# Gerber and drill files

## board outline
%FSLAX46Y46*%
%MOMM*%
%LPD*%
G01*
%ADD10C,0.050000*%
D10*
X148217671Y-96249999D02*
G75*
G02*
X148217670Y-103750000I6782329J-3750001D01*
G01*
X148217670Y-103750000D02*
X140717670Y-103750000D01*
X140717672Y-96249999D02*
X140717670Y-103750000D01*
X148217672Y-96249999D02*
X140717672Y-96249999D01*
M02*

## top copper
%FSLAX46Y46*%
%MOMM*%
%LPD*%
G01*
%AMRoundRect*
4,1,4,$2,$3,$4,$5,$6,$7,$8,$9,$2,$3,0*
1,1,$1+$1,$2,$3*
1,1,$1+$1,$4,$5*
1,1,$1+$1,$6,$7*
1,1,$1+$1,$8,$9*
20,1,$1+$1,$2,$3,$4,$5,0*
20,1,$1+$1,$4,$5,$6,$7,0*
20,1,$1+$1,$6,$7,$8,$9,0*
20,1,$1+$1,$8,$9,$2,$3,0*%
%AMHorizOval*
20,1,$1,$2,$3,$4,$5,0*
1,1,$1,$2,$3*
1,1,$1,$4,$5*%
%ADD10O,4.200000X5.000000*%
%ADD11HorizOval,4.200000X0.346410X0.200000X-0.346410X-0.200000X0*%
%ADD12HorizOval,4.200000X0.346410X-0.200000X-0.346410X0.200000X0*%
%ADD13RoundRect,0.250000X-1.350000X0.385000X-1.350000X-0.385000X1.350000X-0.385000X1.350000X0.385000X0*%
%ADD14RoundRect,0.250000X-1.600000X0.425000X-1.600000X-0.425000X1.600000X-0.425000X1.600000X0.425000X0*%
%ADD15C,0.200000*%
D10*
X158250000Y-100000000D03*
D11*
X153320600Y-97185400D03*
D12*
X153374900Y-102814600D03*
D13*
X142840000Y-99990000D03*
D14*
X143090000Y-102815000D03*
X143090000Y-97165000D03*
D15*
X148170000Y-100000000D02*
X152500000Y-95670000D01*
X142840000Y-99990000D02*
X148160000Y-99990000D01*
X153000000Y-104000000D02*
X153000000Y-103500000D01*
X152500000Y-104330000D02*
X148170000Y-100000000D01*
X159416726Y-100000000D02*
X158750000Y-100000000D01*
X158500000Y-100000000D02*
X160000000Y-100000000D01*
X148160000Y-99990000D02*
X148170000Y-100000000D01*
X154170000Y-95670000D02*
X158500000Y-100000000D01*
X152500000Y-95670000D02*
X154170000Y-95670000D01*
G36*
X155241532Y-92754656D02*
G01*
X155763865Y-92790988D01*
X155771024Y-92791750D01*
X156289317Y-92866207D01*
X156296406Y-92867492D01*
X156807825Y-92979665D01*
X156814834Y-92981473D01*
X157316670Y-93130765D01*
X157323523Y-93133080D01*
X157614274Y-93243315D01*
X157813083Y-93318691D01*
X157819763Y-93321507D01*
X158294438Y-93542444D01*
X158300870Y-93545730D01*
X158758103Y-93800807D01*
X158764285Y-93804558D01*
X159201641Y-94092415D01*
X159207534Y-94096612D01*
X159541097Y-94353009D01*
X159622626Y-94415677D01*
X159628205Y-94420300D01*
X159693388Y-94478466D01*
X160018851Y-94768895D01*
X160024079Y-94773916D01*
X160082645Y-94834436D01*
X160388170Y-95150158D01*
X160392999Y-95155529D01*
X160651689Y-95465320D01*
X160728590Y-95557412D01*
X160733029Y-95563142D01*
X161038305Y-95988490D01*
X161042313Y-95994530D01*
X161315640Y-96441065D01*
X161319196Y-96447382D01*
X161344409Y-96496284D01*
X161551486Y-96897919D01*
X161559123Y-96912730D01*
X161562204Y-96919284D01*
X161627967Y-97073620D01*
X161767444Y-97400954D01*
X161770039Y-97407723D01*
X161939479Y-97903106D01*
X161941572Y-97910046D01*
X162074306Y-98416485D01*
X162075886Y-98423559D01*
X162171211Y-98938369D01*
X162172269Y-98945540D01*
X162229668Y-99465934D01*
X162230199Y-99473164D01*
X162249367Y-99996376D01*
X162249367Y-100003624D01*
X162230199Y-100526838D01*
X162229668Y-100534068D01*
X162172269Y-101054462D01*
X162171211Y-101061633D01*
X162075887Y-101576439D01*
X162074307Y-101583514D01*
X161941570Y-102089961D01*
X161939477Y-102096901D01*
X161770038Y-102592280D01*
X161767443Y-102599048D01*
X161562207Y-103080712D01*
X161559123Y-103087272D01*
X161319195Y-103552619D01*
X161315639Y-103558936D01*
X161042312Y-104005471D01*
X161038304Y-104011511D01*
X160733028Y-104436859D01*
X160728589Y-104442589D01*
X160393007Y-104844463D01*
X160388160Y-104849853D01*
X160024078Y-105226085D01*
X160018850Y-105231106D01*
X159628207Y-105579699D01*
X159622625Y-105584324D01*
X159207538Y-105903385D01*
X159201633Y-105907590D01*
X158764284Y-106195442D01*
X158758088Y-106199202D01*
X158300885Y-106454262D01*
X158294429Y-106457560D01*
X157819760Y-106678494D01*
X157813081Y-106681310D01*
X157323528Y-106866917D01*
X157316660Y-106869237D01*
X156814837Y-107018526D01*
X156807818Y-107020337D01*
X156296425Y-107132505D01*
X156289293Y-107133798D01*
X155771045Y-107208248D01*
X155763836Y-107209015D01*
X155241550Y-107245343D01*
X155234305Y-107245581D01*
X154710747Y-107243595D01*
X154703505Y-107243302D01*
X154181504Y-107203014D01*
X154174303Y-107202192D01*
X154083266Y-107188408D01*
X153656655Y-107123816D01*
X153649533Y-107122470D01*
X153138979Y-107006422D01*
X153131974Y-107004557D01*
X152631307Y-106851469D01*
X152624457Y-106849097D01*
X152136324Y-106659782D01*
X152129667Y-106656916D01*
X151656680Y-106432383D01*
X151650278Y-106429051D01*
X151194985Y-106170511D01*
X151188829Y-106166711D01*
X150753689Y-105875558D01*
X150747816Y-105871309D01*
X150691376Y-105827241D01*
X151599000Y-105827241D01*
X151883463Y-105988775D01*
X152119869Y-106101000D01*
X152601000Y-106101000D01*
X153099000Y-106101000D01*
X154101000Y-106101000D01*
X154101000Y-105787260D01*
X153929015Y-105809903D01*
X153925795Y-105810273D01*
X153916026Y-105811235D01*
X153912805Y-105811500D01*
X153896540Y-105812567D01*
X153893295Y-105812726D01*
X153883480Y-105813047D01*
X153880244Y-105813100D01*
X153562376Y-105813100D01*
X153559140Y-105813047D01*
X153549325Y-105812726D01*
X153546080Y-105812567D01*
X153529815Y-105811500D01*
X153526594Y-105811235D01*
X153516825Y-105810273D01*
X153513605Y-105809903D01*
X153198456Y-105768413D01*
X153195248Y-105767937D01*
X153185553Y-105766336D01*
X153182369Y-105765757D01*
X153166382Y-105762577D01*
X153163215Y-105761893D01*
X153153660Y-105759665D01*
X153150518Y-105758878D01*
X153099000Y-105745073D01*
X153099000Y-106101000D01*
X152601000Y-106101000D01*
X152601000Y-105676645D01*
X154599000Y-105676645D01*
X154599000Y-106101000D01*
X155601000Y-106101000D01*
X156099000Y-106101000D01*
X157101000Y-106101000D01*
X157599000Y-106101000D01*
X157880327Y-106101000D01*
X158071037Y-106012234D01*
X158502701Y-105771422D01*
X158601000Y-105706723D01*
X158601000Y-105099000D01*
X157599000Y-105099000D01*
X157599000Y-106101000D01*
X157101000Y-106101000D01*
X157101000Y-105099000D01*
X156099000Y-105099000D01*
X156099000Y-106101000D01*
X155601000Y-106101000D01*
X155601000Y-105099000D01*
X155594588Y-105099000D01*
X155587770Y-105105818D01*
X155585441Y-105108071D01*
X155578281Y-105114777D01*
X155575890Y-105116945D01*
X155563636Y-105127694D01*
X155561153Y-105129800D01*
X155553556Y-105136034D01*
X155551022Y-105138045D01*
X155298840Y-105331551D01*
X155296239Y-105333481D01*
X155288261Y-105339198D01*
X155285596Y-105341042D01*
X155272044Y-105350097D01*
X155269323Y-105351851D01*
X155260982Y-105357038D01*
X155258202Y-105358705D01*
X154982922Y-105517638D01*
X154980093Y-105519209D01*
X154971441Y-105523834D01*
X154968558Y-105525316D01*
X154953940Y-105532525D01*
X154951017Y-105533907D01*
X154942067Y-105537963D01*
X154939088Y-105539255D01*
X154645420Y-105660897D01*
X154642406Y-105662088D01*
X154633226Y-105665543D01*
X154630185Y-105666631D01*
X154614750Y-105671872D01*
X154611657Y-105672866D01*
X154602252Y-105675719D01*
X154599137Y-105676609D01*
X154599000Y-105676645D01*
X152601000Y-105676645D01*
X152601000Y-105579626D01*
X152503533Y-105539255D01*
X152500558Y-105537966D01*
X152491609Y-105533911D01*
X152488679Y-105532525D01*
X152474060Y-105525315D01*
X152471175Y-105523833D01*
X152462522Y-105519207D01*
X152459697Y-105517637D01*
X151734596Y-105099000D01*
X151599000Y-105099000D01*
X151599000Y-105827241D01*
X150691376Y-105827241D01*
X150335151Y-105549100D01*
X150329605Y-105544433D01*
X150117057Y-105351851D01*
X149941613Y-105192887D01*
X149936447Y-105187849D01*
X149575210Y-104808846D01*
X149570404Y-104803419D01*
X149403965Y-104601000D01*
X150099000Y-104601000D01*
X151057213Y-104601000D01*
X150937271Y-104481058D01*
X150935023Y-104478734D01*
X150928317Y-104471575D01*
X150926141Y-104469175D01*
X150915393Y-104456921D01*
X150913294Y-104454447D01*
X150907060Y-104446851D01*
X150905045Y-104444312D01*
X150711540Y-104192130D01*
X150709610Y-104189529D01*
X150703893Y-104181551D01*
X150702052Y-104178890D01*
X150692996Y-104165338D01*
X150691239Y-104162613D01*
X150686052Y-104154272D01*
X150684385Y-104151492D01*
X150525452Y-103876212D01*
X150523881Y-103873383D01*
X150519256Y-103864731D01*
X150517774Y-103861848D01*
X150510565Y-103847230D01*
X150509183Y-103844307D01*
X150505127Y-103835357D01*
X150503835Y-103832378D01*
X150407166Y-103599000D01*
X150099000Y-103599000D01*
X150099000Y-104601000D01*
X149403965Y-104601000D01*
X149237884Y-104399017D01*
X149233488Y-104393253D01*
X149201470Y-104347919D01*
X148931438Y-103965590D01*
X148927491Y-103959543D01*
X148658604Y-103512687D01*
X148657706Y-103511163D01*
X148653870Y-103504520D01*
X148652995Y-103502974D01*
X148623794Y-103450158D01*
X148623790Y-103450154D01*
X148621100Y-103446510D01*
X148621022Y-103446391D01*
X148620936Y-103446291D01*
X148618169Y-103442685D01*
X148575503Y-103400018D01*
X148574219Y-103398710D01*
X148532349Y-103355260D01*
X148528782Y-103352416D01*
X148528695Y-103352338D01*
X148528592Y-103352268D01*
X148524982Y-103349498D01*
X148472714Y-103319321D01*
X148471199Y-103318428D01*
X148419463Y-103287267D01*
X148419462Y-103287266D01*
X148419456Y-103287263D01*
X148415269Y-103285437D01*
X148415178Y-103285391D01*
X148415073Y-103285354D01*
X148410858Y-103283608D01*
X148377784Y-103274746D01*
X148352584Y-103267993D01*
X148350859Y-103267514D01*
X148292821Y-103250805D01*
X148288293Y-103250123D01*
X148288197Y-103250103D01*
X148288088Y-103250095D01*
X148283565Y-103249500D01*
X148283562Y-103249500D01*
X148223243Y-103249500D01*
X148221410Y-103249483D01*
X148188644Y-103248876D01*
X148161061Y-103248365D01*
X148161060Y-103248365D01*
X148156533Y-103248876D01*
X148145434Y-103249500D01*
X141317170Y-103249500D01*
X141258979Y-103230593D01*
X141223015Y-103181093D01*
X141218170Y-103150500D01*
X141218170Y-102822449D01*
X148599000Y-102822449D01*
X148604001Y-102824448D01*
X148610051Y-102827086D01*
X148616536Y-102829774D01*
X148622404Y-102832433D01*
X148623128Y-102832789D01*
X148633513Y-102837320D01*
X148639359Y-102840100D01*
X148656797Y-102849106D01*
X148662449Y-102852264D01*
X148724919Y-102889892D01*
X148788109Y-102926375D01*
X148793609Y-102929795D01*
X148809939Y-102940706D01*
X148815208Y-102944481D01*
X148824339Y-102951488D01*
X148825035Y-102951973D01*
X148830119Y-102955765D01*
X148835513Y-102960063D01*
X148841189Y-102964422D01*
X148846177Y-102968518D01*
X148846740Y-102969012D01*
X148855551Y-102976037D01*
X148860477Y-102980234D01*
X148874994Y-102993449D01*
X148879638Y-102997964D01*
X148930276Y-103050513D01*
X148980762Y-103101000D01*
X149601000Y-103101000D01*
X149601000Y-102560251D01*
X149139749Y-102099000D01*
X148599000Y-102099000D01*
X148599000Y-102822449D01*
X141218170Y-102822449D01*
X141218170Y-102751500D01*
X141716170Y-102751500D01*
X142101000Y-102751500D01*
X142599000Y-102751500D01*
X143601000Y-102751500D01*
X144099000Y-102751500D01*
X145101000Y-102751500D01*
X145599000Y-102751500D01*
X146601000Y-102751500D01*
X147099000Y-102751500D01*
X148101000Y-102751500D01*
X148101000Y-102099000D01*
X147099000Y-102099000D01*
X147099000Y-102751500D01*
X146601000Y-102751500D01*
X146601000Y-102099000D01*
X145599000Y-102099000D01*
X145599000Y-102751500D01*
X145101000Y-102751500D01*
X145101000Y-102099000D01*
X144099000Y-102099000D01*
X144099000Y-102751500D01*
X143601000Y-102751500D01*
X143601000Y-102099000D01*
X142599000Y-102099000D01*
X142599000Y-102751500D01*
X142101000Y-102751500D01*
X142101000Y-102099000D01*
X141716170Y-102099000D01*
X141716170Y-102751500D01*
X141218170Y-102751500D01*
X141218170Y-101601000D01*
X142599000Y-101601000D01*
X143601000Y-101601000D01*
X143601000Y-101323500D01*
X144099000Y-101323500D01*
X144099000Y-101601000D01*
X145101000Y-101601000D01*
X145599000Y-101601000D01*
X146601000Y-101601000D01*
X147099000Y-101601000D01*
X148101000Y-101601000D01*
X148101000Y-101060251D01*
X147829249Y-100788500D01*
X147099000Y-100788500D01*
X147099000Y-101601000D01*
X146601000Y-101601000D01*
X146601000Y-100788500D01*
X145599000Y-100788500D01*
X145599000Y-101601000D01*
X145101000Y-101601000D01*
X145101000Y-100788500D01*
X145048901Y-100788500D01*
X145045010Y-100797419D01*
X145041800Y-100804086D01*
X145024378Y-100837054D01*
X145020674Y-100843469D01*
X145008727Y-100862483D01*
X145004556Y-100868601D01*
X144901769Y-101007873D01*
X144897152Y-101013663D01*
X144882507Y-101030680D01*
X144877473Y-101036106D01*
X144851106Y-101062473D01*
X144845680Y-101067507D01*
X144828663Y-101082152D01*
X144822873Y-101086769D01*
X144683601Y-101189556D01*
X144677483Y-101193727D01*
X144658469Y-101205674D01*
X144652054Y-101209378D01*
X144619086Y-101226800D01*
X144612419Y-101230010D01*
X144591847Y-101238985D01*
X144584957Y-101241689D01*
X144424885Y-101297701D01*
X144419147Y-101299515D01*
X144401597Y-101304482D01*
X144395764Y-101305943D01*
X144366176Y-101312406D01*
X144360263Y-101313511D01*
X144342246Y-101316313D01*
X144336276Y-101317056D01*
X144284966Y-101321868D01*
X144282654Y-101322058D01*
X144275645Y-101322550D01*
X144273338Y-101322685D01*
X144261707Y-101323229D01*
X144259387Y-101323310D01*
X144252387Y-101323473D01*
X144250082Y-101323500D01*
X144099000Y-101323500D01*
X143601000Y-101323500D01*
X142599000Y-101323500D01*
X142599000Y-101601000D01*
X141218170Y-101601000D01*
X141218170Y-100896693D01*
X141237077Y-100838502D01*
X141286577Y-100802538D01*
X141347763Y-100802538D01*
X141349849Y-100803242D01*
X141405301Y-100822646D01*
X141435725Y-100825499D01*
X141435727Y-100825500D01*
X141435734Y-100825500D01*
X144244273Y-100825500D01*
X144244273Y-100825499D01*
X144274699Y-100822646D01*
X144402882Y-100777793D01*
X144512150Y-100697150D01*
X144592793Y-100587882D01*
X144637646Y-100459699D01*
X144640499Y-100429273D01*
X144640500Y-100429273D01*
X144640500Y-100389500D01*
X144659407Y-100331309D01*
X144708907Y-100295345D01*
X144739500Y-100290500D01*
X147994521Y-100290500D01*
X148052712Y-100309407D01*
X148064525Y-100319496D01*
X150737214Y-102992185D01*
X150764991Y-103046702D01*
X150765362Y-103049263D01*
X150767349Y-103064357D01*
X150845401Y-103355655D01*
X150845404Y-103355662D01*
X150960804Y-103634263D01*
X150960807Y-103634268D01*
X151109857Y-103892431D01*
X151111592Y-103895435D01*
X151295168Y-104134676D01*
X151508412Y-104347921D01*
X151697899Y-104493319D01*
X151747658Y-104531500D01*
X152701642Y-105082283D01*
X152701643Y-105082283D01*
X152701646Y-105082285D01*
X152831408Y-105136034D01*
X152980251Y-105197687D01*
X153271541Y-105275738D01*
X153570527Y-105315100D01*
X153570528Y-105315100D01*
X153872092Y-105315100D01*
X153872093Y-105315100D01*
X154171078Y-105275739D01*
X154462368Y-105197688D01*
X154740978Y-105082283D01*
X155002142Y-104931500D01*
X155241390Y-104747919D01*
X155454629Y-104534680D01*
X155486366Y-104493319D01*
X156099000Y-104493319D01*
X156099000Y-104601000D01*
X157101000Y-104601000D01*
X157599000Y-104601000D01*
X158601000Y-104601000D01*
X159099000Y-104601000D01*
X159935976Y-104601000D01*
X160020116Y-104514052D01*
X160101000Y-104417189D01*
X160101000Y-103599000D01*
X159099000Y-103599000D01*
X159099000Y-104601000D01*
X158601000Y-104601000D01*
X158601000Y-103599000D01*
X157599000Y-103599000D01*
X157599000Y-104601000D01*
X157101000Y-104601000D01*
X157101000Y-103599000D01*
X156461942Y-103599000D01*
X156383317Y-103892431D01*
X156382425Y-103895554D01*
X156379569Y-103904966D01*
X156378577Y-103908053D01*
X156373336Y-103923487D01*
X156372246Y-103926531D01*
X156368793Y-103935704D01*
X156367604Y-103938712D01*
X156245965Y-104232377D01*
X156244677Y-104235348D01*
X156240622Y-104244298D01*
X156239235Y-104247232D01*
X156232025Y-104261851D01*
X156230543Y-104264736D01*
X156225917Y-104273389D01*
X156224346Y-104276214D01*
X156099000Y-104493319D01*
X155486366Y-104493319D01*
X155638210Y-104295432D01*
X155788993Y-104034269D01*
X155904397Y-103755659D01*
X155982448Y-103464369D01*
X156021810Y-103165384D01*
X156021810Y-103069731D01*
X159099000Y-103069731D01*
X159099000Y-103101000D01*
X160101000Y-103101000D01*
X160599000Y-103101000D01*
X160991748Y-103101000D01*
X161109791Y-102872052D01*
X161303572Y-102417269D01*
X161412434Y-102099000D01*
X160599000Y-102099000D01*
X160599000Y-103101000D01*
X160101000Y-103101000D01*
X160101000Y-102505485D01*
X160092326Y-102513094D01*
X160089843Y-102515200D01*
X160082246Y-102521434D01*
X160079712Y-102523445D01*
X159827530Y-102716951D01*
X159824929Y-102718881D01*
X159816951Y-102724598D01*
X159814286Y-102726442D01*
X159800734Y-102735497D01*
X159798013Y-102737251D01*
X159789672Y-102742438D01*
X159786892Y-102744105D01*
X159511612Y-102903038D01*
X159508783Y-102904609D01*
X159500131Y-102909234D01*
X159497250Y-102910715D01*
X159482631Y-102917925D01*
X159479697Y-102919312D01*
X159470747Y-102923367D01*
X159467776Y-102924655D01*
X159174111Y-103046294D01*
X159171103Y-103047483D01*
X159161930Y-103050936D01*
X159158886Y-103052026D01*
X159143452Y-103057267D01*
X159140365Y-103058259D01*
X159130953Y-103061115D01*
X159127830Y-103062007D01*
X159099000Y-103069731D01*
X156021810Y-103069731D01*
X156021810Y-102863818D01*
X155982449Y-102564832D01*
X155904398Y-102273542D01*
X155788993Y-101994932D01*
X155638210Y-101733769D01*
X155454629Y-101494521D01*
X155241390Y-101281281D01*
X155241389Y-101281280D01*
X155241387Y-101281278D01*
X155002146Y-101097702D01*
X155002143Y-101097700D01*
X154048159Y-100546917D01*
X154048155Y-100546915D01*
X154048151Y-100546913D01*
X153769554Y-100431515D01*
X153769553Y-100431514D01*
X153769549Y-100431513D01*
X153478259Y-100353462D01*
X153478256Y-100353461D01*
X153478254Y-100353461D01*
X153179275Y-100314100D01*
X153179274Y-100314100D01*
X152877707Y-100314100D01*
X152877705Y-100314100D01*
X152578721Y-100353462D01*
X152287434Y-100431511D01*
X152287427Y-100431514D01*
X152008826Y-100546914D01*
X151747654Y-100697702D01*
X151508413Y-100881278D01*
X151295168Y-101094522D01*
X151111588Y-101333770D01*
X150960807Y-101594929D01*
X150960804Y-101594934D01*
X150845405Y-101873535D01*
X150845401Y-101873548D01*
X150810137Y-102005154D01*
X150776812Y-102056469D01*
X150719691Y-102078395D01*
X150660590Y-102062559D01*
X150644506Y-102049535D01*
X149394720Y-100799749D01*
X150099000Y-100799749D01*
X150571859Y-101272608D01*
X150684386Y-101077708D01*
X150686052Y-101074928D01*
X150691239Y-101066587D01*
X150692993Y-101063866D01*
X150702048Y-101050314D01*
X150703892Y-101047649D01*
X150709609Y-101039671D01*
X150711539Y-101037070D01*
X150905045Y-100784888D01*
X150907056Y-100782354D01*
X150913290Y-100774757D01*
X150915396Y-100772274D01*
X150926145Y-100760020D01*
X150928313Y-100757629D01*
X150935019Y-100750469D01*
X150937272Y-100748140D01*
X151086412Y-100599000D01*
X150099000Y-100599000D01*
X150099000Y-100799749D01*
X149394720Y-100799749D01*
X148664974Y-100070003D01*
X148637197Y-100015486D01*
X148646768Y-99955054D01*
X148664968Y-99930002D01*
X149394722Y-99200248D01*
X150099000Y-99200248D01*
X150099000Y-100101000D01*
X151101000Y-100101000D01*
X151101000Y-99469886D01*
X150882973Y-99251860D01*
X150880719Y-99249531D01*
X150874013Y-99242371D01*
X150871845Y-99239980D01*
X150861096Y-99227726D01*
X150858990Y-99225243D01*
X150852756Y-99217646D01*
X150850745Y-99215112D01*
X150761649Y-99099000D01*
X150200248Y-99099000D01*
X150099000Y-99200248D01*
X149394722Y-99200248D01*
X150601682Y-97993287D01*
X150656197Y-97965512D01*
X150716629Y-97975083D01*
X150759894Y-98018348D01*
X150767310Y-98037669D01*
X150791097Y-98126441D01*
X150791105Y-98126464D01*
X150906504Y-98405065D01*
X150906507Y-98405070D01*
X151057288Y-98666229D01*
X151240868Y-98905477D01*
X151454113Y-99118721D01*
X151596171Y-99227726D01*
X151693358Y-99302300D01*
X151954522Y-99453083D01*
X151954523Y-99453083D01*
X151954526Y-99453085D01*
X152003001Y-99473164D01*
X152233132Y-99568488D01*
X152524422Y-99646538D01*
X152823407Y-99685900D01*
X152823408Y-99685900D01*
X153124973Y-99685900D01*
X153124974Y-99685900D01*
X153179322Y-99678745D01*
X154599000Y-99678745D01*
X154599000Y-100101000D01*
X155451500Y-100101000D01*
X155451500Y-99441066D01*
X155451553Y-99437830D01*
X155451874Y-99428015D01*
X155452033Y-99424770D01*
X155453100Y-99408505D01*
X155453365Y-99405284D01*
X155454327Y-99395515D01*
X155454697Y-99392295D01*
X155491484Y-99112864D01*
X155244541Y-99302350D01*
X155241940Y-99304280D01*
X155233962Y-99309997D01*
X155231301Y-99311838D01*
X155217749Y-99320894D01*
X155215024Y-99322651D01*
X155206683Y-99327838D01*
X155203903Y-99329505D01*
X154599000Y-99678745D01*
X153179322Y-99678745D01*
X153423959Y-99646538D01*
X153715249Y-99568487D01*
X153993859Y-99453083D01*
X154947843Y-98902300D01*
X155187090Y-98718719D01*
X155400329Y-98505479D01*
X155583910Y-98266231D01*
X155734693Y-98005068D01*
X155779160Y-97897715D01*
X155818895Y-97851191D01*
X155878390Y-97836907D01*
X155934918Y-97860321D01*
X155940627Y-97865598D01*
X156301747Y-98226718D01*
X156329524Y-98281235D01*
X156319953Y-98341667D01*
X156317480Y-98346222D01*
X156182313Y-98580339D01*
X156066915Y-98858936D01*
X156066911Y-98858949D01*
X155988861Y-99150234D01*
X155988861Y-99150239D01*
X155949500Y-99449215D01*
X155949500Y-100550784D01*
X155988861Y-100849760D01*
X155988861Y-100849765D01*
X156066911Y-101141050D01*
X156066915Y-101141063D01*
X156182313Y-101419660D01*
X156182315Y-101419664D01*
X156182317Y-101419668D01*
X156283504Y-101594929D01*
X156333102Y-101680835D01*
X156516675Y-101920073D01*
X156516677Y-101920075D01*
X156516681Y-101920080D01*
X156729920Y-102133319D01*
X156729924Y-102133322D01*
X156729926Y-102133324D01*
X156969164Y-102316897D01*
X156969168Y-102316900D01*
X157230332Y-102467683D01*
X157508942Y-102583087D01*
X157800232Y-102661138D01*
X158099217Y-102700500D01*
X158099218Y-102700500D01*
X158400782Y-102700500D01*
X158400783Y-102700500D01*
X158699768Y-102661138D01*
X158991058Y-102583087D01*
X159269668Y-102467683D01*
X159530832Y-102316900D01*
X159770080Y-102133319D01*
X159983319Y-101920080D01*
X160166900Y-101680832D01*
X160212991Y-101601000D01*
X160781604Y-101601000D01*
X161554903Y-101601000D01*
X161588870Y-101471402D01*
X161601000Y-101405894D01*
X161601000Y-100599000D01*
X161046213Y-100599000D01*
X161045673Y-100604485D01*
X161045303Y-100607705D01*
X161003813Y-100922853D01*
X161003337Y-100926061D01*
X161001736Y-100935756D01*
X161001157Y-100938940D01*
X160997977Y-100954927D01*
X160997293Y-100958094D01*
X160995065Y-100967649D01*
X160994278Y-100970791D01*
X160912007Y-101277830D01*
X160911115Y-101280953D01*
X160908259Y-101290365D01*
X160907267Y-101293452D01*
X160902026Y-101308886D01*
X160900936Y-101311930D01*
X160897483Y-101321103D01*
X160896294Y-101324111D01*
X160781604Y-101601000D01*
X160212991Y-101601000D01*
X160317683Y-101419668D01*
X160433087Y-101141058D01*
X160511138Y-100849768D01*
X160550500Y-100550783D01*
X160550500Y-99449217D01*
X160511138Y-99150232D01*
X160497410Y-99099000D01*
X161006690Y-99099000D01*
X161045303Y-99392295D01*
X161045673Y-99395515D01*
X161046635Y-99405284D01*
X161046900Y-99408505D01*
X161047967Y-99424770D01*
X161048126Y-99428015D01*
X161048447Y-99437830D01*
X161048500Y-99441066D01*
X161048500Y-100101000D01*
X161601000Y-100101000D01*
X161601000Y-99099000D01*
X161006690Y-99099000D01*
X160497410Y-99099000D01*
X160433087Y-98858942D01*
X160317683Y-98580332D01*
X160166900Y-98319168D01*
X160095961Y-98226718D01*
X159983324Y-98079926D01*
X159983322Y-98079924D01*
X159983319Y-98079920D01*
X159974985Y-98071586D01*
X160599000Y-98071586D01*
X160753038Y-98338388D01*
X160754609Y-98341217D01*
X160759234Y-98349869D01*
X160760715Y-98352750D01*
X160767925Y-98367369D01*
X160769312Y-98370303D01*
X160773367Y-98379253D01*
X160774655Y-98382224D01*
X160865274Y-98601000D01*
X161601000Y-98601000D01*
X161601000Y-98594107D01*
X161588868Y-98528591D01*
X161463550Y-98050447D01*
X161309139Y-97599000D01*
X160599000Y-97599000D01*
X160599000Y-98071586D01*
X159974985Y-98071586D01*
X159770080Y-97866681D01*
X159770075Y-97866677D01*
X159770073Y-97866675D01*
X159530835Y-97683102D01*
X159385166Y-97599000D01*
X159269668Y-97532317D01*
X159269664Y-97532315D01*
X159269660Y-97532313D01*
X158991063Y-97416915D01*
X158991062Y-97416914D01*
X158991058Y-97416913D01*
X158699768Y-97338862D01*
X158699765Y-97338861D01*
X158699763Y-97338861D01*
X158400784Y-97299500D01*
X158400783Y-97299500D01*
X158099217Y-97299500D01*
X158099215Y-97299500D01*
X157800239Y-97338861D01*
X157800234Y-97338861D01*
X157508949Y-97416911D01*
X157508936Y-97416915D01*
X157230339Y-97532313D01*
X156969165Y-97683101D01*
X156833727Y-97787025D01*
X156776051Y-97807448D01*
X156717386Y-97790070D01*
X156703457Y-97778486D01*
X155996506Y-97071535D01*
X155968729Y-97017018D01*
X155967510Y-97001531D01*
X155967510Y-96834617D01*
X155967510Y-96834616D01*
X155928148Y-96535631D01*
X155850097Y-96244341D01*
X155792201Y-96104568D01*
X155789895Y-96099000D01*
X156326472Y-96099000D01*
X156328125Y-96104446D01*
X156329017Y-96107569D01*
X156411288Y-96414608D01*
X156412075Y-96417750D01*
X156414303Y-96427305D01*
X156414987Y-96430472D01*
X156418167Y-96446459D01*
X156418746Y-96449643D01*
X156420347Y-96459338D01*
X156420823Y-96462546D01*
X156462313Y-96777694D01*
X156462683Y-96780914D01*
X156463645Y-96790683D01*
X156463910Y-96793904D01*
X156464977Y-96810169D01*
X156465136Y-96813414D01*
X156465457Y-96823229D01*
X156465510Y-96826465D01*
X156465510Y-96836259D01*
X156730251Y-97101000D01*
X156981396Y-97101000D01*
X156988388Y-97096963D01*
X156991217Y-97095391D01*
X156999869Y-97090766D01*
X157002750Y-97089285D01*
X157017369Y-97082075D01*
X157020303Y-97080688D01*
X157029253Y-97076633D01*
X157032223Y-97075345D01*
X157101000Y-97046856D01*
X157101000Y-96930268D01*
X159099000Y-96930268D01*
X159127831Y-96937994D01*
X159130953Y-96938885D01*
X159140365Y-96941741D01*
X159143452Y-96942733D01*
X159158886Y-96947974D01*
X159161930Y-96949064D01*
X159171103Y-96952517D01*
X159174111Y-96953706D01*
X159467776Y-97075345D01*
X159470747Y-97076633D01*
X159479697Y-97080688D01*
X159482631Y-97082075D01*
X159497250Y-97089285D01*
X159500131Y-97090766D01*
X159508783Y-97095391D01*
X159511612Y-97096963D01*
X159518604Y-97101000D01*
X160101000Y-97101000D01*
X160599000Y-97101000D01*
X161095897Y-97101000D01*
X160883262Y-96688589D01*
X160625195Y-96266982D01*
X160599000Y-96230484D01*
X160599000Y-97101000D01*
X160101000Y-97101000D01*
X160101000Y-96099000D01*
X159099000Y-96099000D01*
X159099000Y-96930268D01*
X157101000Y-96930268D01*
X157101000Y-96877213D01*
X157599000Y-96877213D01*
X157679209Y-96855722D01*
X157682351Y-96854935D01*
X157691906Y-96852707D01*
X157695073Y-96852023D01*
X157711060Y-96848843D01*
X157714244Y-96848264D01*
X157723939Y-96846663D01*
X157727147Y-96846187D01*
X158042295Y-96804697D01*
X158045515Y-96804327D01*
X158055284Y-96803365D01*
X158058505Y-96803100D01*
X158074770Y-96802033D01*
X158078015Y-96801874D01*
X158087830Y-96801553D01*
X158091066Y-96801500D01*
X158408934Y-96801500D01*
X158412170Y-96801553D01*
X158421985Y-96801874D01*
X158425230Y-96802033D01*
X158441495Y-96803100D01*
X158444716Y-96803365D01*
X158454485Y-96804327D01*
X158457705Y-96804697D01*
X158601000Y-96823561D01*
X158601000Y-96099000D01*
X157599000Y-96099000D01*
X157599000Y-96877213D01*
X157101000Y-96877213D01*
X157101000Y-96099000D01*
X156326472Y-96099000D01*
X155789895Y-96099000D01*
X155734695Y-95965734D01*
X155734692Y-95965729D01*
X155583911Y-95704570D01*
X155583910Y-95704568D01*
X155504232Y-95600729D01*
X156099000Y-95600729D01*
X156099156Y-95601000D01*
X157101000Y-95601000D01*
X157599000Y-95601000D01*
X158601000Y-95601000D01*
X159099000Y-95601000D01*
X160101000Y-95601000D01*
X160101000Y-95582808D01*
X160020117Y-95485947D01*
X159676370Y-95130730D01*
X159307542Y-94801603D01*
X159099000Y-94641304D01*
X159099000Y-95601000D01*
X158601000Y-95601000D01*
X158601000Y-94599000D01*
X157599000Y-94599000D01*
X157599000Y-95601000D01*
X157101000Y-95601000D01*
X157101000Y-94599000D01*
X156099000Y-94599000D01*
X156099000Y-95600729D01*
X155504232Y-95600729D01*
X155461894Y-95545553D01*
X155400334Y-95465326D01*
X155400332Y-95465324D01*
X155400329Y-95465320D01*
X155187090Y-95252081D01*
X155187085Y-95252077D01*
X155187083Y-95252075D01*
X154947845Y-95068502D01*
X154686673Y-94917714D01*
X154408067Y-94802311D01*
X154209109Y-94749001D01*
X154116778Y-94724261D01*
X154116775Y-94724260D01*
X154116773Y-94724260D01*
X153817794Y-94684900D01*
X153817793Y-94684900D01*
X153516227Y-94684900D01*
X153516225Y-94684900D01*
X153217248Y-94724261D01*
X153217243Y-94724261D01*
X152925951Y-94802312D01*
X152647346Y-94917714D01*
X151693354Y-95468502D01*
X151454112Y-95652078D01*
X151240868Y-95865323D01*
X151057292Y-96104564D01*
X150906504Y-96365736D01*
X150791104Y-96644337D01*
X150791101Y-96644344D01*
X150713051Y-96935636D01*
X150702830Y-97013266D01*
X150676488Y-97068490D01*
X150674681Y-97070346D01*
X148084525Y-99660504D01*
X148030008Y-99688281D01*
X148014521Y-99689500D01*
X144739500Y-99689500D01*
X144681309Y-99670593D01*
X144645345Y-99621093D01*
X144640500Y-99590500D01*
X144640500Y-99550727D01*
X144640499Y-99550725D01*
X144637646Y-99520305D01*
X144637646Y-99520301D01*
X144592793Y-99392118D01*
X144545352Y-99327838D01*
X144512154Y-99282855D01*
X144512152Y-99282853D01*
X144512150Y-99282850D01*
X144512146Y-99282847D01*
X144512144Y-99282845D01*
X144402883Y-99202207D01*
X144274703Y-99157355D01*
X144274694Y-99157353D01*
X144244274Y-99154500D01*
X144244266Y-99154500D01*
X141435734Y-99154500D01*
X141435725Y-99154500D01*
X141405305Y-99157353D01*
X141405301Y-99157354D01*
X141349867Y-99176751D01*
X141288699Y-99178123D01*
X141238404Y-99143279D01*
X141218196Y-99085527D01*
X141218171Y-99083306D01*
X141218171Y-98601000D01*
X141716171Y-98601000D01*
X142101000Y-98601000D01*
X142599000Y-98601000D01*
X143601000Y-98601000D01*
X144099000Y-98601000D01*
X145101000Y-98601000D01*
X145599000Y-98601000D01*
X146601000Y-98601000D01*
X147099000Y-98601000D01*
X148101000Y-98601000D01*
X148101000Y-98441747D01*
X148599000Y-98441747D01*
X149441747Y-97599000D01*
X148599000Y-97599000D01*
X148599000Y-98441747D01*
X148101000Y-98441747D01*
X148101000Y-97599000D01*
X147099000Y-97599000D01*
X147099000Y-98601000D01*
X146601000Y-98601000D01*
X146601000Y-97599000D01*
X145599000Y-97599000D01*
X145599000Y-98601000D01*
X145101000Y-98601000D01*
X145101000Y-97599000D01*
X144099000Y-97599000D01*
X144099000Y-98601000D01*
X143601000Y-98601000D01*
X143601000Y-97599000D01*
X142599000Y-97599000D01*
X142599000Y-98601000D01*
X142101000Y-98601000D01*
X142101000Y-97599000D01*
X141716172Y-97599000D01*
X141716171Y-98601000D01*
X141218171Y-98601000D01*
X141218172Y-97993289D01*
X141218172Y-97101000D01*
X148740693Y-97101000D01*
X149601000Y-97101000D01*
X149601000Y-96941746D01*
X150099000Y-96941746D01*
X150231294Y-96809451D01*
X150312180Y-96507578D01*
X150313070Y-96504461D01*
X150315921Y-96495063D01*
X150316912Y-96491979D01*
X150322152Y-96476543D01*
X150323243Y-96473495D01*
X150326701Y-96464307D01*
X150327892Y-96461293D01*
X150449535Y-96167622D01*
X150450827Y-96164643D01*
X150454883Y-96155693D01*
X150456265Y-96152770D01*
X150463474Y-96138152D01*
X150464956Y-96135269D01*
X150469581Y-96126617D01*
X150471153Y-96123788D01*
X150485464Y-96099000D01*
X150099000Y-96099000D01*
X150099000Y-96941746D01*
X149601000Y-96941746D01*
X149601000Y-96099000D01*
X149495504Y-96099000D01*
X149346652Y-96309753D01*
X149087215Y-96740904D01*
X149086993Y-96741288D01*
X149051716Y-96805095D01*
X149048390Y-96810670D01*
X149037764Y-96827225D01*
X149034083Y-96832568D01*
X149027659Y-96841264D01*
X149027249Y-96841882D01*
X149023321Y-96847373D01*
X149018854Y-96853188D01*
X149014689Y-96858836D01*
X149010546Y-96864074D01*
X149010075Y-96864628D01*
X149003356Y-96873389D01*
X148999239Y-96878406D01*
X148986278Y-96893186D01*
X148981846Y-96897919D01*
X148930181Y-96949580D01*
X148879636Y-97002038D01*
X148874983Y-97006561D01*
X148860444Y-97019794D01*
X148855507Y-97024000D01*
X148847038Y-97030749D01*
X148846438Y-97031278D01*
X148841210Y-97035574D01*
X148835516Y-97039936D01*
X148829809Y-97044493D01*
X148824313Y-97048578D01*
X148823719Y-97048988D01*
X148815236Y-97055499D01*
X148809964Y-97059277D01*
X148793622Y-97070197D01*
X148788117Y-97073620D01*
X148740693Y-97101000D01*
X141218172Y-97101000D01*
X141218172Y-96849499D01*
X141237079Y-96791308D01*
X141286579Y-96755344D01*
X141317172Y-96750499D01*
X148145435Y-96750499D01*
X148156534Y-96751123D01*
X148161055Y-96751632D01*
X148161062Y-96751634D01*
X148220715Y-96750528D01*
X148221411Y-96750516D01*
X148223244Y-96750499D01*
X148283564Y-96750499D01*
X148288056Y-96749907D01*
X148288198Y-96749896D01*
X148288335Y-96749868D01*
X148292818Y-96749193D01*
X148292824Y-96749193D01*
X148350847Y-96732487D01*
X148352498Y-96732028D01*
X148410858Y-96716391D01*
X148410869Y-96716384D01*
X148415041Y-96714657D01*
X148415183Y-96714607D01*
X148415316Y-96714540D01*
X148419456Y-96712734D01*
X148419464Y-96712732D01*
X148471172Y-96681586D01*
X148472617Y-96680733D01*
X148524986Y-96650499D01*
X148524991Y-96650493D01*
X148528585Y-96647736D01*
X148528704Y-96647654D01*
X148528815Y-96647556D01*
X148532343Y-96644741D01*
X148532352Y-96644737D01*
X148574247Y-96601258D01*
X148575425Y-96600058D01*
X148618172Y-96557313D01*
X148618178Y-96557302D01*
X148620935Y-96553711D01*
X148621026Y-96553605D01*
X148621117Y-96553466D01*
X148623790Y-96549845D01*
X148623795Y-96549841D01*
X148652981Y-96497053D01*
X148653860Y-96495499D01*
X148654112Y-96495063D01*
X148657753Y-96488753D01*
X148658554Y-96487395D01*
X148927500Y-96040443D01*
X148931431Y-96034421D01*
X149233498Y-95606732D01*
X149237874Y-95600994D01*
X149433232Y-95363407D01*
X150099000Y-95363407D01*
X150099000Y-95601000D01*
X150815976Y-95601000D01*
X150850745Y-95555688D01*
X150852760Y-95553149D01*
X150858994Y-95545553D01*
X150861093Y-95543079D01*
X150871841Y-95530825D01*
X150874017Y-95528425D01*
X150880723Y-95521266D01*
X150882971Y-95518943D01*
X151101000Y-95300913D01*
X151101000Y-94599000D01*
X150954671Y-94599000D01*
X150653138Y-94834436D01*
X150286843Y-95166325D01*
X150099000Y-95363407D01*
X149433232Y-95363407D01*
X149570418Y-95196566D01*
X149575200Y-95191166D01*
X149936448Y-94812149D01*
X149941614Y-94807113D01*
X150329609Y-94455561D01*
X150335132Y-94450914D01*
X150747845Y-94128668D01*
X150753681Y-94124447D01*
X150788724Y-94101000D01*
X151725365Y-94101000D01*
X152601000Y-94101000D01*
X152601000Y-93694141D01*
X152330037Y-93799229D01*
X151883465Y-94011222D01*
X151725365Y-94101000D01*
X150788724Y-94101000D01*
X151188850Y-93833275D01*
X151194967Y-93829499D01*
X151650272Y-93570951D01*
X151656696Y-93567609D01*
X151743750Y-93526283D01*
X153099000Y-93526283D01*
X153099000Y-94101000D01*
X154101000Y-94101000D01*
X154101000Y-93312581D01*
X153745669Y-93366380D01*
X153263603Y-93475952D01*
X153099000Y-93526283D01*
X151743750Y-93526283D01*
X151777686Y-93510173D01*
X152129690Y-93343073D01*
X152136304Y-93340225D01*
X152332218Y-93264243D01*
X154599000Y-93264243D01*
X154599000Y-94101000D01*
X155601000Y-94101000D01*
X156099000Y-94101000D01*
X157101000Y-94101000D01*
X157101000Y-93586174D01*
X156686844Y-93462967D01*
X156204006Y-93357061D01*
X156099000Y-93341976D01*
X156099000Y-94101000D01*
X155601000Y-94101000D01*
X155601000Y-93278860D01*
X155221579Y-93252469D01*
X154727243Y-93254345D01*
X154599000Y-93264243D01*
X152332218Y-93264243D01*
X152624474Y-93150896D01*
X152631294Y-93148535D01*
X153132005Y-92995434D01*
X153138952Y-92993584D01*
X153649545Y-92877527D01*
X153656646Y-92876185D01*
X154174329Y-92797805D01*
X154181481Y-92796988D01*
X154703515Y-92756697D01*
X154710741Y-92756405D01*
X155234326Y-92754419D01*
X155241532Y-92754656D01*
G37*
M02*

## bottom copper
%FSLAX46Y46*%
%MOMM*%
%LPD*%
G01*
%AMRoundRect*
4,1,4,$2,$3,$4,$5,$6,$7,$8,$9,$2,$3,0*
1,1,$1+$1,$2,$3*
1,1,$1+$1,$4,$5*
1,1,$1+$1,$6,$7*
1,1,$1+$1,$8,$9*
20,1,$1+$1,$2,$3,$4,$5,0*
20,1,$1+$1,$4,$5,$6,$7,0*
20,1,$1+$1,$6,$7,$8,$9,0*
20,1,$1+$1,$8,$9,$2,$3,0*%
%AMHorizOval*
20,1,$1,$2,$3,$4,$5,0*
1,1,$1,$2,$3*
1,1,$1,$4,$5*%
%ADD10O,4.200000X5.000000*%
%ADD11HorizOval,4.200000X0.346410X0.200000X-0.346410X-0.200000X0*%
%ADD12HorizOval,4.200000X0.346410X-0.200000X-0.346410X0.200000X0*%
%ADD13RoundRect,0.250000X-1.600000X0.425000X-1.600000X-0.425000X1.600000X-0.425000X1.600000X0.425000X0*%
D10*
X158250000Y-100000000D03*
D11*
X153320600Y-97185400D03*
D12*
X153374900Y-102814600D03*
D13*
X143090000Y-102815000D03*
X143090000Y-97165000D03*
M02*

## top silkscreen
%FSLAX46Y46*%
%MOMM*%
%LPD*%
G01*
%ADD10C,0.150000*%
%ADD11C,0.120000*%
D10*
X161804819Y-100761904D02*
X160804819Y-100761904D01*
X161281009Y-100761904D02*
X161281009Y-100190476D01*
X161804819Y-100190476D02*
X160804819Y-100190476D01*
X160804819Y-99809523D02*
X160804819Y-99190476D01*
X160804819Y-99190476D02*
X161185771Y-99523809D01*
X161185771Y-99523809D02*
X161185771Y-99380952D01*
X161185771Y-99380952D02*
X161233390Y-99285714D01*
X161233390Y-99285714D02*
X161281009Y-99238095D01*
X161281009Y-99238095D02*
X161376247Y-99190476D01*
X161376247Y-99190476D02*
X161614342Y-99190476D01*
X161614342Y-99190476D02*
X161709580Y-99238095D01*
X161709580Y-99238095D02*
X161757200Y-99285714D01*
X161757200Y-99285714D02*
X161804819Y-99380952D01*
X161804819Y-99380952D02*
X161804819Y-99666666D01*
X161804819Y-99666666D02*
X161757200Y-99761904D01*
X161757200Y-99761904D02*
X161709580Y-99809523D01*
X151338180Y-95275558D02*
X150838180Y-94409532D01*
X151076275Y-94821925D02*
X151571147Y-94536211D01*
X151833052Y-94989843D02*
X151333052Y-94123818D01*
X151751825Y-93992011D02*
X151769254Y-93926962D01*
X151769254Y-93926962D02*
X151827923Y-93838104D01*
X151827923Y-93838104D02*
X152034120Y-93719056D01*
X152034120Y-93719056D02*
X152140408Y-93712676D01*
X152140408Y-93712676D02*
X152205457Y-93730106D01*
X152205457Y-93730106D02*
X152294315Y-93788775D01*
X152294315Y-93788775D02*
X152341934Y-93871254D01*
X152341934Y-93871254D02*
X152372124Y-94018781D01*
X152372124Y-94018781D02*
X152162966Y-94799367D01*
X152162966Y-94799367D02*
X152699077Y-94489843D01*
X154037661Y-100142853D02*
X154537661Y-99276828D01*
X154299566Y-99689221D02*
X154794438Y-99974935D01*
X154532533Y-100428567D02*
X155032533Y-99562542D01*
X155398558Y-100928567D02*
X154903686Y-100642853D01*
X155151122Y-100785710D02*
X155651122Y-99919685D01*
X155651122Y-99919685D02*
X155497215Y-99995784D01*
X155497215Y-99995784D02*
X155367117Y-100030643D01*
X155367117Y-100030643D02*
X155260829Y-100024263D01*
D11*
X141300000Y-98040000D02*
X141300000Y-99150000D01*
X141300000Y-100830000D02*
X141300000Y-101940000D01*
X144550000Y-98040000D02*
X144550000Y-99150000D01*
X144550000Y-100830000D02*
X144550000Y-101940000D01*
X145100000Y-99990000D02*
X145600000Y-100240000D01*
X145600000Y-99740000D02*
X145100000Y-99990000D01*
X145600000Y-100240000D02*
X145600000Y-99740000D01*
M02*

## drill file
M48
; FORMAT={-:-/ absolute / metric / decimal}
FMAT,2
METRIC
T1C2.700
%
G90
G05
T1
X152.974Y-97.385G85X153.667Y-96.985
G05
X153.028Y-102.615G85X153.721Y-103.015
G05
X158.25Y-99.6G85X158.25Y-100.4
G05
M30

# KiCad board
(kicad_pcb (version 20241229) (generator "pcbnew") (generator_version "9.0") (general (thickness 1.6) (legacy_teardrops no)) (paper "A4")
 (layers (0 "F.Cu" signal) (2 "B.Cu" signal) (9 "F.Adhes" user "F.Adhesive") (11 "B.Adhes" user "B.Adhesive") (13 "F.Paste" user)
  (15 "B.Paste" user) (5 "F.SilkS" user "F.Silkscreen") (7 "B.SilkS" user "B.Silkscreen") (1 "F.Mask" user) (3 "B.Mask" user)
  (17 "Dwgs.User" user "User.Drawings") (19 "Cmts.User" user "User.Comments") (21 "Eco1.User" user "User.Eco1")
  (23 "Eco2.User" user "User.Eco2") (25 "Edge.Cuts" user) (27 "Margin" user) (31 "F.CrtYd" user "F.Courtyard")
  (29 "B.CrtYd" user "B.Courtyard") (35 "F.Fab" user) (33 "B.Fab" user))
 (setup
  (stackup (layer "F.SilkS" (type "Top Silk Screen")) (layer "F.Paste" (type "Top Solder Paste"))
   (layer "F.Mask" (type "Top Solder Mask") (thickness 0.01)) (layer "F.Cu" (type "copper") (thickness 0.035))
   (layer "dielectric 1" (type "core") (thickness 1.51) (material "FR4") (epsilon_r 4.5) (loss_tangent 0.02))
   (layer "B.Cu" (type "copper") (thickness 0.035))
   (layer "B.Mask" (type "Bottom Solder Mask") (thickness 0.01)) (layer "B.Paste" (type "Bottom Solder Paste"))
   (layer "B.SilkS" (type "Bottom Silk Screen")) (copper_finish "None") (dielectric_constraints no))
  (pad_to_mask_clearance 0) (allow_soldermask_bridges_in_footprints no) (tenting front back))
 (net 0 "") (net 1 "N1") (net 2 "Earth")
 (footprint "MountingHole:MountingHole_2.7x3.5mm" (layer "F.Cu") (at 158.25 100 -90)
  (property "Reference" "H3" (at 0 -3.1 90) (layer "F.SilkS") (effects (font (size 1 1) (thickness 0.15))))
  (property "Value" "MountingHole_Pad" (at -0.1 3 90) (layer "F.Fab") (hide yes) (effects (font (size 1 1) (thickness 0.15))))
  (pad "1" thru_hole oval (at 0 0 270) (size 5 4.2) (drill oval 3.5 2.7) (layers "*.Cu" "*.Mask") (remove_unused_layers no) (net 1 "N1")))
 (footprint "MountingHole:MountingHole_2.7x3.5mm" (layer "F.Cu") (at 153.3206 97.1854 30)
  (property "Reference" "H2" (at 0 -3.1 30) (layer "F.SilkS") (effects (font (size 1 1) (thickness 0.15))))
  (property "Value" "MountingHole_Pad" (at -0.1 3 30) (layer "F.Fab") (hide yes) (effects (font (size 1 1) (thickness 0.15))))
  (pad "1" thru_hole oval (at 0 0 30) (size 5 4.2) (drill oval 3.5 2.7) (layers "*.Cu" "*.Mask") (remove_unused_layers no) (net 1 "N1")))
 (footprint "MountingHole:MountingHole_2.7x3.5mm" (layer "F.Cu") (at 153.3749 102.8146 -30)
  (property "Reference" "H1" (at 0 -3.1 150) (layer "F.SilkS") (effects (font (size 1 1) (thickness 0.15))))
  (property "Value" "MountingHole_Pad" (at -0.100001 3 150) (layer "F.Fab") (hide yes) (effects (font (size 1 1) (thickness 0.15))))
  (pad "1" thru_hole oval (at 0 0 330) (size 5 4.2) (drill oval 3.5 2.7) (layers "*.Cu" "*.Mask") (remove_unused_layers no) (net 1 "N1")))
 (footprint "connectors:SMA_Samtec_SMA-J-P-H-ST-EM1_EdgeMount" (layer "F.Cu") (at 142.84 99.99 180)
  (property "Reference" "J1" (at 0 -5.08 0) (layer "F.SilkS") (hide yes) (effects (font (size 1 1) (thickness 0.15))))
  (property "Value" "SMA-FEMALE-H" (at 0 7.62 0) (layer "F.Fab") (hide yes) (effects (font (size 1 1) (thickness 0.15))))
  (fp_line (start 1.54 1.95) (end 1.54 0.84) (stroke (width 0.12) (type solid)) (layer "F.SilkS"))
  (fp_line (start 1.54 -0.84) (end 1.54 -1.95) (stroke (width 0.12) (type solid)) (layer "F.SilkS"))
  (fp_line (start -1.71 1.95) (end -1.71 0.84) (stroke (width 0.12) (type solid)) (layer "F.SilkS"))
  (fp_line (start -1.71 -0.84) (end -1.71 -1.95) (stroke (width 0.12) (type solid)) (layer "F.SilkS"))
  (fp_line (start -2.26 0) (end -2.76 -0.25) (stroke (width 0.12) (type solid)) (layer "F.SilkS"))
  (fp_line (start -2.76 0.25) (end -2.26 0) (stroke (width 0.12) (type solid)) (layer "F.SilkS"))
  (fp_line (start -2.76 -0.25) (end -2.76 0.25) (stroke (width 0.12) (type solid)) (layer "F.SilkS"))
  (pad "1" smd roundrect (at 0 0 270) (size 1.27 3.2) (layers "F.Cu" "F.Mask") (roundrect_rratio 0.1968503937) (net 1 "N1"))
  (pad "2" smd roundrect (at -0.25 -2.825 270) (size 1.35 3.7) (layers "F.Cu" "F.Mask") (roundrect_rratio 0.1851851852) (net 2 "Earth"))
  (pad "2" smd roundrect (at -0.25 -2.825 270) (size 1.35 3.7) (layers "B.Cu" "B.Mask") (roundrect_rratio 0.1851851852) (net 2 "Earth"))
  (pad "2" smd roundrect (at -0.25 2.825 270) (size 1.35 3.7) (layers "F.Cu" "F.Mask") (roundrect_rratio 0.1851851852) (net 2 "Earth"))
  (pad "2" smd roundrect (at -0.25 2.825 270) (size 1.35 3.7) (layers "B.Cu" "B.Mask") (roundrect_rratio 0.1851851852) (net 2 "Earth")))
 (gr_arc (start 148.217671 96.249999) (mid 162.75 100.000001) (end 148.21767 103.75) (stroke (width 0.05) (type default))
  (layer "Edge.Cuts"))
 (gr_line (start 148.21767 103.75) (end 140.71767 103.75) (stroke (width 0.05) (type solid)) (layer "Edge.Cuts"))
 (gr_line (start 140.717672 96.249999) (end 140.71767 103.75) (stroke (width 0.05) (type default)) (layer "Edge.Cuts"))
 (gr_line (start 148.217672 96.249999) (end 140.717672 96.249999) (stroke (width 0.05) (type solid)) (layer "Edge.Cuts"))
 (segment (start 148.17 100) (end 152.5 95.67) (width 0.2) (layer "F.Cu") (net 1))
 (segment (start 142.84 99.99) (end 148.16 99.99) (width 0.2) (layer "F.Cu") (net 1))
 (segment (start 153 104) (end 153 103.5) (width 0.2) (layer "F.Cu") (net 1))
 (segment (start 152.5 104.33) (end 148.17 100) (width 0.2) (layer "F.Cu") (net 1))
 (segment (start 159.416726 100) (end 158.75 100) (width 0.2) (layer "F.Cu") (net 1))
 (segment (start 158.5 100) (end 160 100) (width 0.2) (layer "F.Cu") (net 1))
 (segment (start 148.16 99.99) (end 148.17 100) (width 0.2) (layer "F.Cu") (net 1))
 (segment (start 154.17 95.67) (end 158.5 100) (width 0.2) (layer "F.Cu") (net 1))
 (segment (start 152.5 95.67) (end 154.17 95.67) (width 0.2) (layer "F.Cu") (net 1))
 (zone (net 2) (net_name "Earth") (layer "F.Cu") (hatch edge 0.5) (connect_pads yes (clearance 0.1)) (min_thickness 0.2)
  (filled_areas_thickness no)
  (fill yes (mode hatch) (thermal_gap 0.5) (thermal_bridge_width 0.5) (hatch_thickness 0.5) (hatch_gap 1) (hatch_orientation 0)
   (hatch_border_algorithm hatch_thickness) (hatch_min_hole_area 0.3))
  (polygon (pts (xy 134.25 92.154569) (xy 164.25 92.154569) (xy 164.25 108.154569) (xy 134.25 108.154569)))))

